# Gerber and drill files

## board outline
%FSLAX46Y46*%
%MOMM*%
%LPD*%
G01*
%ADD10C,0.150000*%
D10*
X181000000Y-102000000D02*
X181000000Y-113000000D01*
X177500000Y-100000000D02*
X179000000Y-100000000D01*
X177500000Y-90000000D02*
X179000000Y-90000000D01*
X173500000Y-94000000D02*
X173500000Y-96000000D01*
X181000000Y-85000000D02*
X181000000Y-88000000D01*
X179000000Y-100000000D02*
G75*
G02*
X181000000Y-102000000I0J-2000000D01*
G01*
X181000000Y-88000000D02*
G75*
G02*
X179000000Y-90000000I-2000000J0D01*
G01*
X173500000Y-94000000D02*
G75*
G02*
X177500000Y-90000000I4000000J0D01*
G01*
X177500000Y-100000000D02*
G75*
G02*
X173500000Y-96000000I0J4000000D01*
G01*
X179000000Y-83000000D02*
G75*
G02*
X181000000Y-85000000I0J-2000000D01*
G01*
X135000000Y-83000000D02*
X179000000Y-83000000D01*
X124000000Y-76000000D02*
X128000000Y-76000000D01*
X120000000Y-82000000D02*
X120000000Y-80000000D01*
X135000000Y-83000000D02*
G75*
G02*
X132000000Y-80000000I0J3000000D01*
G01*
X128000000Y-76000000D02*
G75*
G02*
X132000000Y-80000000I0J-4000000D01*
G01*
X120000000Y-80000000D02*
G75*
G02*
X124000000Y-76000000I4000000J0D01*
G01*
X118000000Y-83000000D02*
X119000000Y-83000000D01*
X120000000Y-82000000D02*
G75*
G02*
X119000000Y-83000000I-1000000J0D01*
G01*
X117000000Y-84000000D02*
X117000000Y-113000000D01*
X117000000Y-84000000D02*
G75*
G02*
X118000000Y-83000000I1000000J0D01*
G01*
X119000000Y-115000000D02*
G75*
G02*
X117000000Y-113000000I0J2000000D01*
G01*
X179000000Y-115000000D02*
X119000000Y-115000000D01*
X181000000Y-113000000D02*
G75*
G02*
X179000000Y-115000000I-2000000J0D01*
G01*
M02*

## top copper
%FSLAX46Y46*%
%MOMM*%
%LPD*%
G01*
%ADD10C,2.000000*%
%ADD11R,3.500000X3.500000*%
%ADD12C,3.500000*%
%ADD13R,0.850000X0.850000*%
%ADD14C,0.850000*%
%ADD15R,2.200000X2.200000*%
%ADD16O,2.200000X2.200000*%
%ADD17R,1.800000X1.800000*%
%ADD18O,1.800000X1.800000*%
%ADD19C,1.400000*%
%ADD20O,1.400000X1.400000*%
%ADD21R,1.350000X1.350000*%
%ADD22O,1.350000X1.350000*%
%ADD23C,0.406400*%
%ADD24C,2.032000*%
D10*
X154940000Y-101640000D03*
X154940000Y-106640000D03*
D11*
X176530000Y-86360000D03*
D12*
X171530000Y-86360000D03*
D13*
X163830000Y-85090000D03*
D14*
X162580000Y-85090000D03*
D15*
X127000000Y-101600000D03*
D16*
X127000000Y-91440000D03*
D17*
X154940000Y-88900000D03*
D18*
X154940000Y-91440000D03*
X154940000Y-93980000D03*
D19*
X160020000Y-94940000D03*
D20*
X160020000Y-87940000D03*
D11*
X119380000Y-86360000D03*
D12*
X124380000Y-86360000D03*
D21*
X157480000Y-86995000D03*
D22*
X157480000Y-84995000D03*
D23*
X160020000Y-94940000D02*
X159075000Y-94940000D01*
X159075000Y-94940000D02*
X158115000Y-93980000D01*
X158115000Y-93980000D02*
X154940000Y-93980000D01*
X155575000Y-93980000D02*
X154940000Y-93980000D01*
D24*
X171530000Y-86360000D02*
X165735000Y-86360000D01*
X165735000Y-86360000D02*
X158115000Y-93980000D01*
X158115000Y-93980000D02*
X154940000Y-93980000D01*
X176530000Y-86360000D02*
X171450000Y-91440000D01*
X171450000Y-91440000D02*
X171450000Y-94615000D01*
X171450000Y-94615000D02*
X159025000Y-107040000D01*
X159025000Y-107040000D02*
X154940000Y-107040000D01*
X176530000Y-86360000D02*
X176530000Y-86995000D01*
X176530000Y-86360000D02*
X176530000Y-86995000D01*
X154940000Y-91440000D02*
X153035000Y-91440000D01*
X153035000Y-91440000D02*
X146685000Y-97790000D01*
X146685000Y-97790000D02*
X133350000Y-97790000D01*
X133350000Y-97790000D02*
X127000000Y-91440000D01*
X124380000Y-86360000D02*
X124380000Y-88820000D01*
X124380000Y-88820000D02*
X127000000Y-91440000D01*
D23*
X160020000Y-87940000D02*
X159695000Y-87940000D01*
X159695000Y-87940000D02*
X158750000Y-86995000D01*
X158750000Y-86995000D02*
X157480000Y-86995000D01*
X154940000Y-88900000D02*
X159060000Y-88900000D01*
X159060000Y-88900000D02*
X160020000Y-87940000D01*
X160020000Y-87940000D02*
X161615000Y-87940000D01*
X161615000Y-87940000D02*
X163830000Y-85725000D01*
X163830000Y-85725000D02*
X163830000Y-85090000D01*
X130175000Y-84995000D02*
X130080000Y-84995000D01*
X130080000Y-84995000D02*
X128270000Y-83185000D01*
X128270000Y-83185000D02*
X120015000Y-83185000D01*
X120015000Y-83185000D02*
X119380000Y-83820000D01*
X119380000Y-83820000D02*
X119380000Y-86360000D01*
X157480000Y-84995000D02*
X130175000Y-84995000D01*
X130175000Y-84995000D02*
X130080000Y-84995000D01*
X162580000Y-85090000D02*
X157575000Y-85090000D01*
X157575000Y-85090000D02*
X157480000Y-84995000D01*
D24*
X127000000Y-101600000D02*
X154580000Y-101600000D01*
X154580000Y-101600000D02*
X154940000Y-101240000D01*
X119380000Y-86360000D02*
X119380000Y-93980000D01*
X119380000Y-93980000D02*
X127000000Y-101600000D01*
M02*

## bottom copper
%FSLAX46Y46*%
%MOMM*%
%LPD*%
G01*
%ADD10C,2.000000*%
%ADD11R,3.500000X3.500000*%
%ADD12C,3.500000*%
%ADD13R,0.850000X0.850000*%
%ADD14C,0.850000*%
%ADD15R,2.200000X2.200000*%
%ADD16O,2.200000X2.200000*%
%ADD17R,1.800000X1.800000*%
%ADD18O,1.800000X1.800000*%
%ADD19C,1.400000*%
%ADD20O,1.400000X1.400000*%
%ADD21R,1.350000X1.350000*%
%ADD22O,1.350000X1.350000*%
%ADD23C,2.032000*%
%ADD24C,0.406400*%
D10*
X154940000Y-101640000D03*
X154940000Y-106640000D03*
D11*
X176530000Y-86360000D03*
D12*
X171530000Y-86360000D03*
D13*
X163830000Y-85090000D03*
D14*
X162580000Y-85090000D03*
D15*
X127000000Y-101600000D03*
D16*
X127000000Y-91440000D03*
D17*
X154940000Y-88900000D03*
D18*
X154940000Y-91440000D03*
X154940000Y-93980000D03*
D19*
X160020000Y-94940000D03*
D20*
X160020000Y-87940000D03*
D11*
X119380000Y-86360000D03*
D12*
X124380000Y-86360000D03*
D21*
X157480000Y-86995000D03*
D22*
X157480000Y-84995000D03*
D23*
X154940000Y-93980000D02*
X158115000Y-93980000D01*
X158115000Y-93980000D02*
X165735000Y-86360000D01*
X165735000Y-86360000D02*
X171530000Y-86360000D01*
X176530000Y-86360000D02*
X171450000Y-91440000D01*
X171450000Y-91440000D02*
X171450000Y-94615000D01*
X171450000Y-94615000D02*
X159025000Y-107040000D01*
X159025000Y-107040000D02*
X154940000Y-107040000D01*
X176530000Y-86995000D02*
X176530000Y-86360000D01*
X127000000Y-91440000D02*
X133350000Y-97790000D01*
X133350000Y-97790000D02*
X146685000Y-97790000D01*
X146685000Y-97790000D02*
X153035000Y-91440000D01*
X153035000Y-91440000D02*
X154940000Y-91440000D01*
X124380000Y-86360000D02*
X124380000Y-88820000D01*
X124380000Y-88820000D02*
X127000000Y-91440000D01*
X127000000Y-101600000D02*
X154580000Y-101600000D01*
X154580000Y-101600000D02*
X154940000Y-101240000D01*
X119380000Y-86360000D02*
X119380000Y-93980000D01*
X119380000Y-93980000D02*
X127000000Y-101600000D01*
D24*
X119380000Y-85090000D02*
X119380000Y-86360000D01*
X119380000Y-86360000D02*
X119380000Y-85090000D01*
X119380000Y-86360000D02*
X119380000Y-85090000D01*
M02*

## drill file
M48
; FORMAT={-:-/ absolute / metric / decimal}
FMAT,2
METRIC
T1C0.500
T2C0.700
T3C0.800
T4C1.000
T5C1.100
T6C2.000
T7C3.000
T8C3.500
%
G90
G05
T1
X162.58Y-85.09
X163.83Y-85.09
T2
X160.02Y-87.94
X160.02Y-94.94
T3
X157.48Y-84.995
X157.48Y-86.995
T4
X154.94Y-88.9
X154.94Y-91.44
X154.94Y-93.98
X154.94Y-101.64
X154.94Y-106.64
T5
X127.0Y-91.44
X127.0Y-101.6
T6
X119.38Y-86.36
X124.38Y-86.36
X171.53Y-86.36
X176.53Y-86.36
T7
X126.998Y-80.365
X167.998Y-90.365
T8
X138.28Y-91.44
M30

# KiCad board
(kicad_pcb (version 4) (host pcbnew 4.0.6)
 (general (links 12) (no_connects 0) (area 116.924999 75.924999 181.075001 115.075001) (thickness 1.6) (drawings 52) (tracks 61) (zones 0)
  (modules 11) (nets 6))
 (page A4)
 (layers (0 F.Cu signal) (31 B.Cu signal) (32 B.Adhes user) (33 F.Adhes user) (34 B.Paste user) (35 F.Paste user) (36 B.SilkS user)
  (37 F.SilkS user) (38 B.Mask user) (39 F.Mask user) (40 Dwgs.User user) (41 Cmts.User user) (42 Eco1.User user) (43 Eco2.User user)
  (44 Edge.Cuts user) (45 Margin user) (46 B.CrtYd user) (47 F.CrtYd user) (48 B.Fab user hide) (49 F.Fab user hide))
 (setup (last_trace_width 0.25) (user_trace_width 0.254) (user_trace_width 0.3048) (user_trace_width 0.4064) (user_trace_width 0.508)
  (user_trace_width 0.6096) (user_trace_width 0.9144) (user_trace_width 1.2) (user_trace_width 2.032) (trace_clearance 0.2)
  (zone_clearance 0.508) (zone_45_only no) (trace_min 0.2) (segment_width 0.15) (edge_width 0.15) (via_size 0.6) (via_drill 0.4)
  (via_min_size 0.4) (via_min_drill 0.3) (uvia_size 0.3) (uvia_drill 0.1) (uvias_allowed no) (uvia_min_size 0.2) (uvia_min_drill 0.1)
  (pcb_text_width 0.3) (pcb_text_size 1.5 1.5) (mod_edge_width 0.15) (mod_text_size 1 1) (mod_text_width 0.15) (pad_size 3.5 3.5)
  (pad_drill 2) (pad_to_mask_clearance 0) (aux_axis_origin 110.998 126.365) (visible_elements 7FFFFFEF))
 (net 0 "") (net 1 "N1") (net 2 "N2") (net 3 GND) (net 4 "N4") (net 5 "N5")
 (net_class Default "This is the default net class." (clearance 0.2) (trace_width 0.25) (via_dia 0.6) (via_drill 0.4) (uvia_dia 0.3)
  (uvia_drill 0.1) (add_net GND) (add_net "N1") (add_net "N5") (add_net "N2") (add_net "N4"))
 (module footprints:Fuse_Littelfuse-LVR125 (layer B.Cu) (at 154.94 104.14 270)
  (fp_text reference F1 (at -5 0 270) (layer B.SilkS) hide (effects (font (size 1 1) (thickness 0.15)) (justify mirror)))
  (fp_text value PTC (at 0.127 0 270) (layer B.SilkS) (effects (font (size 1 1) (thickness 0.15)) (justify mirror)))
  (pad 1 thru_hole circle (at -2.5 0 270) (size 2 2) (drill 1) (layers *.Cu *.Mask) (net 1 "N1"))
  (pad 2 thru_hole circle (at 2.5 0 270) (size 2 2) (drill 1) (layers *.Cu *.Mask) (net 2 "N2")))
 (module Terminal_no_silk (layer B.Cu) (at 176.53 86.36 180)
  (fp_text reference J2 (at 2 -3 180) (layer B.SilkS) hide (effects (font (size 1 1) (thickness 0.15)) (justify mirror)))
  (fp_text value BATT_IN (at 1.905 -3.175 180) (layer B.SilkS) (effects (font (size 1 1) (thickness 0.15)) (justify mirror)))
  (pad 1 thru_hole rect (at 0 0 180) (size 3.5 3.5) (drill 2) (layers *.Cu *.Mask) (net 2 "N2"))
  (pad 2 thru_hole circle (at 5 0 180) (size 3.5 3.5) (drill 2) (layers *.Cu *.Mask) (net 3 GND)))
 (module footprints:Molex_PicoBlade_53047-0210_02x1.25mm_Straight (layer F.Cu) (at 163.83 85.09 180)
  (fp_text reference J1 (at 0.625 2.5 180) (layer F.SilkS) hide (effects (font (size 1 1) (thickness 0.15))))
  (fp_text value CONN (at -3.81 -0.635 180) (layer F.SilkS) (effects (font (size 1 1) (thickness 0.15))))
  (pad 1 thru_hole rect (at 0 0 180) (size 0.85 0.85) (drill 0.5) (layers *.Cu *.Mask) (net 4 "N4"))
  (pad 2 thru_hole circle (at 1.25 0 180) (size 0.85 0.85) (drill 0.5) (layers *.Cu *.Mask) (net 1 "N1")))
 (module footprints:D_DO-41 (layer B.Cu) (at 127 101.6 90)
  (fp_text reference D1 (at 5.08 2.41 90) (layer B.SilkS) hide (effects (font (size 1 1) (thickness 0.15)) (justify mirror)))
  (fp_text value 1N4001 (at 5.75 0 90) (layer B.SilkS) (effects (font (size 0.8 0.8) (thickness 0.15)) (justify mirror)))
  (pad 1 thru_hole rect (at 0 0 90) (size 2.2 2.2) (drill 1.1) (layers *.Cu *.Mask) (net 1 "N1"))
  (pad 2 thru_hole oval (at 10.16 0 90) (size 2.2 2.2) (drill 1.1) (layers *.Cu *.Mask) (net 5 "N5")))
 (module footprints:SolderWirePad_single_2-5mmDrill (layer F.Cu) (at 167.998 90.365)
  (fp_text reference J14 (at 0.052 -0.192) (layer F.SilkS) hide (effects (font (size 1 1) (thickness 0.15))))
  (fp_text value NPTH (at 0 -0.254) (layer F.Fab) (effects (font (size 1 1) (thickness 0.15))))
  (pad "" np_thru_hole circle (at 0 0) (size 3 3) (drill 3) (layers *.Cu *.Mask)))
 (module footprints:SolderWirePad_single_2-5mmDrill (layer F.Cu) (at 126.998 80.365)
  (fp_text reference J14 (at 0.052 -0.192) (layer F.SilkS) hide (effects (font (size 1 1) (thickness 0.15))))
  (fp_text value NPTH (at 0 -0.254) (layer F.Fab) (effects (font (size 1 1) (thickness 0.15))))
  (pad "" np_thru_hole circle (at 0 0) (size 3 3) (drill 3) (layers *.Cu *.Mask)))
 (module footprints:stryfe (layer F.Cu) (at 147.32 109.855)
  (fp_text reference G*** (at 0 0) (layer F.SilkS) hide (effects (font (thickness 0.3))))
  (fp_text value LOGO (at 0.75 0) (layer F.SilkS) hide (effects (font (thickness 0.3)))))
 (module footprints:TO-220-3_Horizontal (layer B.Cu) (at 154.94 88.9 270)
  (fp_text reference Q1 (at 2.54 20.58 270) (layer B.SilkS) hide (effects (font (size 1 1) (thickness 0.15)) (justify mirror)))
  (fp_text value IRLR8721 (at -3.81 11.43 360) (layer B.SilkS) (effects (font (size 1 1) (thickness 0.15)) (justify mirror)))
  (pad 0 np_thru_hole oval (at 2.54 16.66 270) (size 3.5 3.5) (drill 3.5) (layers *.Cu *.Mask))
  (pad 1 thru_hole rect (at 0 0 270) (size 1.8 1.8) (drill 1) (layers *.Cu *.Mask) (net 4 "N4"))
  (pad 2 thru_hole oval (at 2.54 0 270) (size 1.8 1.8) (drill 1) (layers *.Cu *.Mask) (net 5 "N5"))
  (pad 3 thru_hole oval (at 5.08 0 270) (size 1.8 1.8) (drill 1) (layers *.Cu *.Mask) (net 3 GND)))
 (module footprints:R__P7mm (layer B.Cu) (at 160.02 91.44 90)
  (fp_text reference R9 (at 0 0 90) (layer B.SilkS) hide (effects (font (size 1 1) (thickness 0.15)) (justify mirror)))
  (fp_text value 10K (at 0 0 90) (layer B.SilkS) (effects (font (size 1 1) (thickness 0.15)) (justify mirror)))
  (pad 1 thru_hole circle (at -3.5 0 90) (size 1.4 1.4) (drill 0.7) (layers *.Cu *.Mask) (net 3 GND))
  (pad 2 thru_hole oval (at 3.5 0 90) (size 1.4 1.4) (drill 0.7) (layers *.Cu *.Mask) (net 4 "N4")))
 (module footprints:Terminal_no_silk (layer B.Cu) (at 119.38 86.36)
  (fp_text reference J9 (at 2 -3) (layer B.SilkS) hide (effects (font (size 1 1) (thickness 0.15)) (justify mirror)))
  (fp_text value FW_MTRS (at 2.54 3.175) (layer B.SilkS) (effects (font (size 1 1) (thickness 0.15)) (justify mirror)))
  (pad 1 thru_hole rect (at 0 0) (size 3.5 3.5) (drill 2) (layers *.Cu *.Mask) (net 1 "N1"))
  (pad 2 thru_hole circle (at 5 0) (size 3.5 3.5) (drill 2) (layers *.Cu *.Mask) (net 5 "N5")))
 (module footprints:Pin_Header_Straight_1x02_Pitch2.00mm (layer F.Cu) (at 157.48 86.995 180)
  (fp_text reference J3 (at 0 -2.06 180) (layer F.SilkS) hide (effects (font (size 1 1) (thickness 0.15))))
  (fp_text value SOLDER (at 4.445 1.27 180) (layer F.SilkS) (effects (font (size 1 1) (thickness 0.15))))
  (pad 1 thru_hole rect (at 0 0 180) (size 1.35 1.35) (drill 0.8) (layers *.Cu *.Mask) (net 4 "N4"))
  (pad 2 thru_hole oval (at 0 2 180) (size 1.35 1.35) (drill 0.8) (layers *.Cu *.Mask) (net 1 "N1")))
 (gr_line (start 181 102) (end 181 113) (angle 90) (layer Edge.Cuts) (width 0.15))
 (gr_line (start 177.5 100) (end 179 100) (angle 90) (layer Edge.Cuts) (width 0.15))
 (gr_line (start 177.5 90) (end 179 90) (angle 90) (layer Edge.Cuts) (width 0.15))
 (gr_line (start 173.5 94) (end 173.5 96) (angle 90) (layer Edge.Cuts) (width 0.15))
 (gr_line (start 181 85) (end 181 88) (angle 90) (layer Edge.Cuts) (width 0.15))
 (gr_arc (start 179 102) (end 179 100) (angle 90) (layer Edge.Cuts) (width 0.15))
 (gr_arc (start 179 88) (end 181 88) (angle 90) (layer Edge.Cuts) (width 0.15))
 (gr_arc (start 177.5 94) (end 173.5 94) (angle 90) (layer Edge.Cuts) (width 0.15))
 (gr_arc (start 177.5 96) (end 177.5 100) (angle 90) (layer Edge.Cuts) (width 0.15))
 (gr_arc (start 179 85) (end 179 83) (angle 90) (layer Edge.Cuts) (width 0.15))
 (gr_line (start 135 83) (end 179 83) (angle 90) (layer Edge.Cuts) (width 0.15))
 (gr_line (start 124 76) (end 128 76) (angle 90) (layer Edge.Cuts) (width 0.15))
 (gr_line (start 120 82) (end 120 80) (angle 90) (layer Edge.Cuts) (width 0.15))
 (gr_arc (start 135 80) (end 135 83) (angle 90) (layer Edge.Cuts) (width 0.15))
 (gr_arc (start 128 80) (end 128 76) (angle 90) (layer Edge.Cuts) (width 0.15))
 (gr_arc (start 124 80) (end 120 80) (angle 90) (layer Edge.Cuts) (width 0.15))
 (gr_line (start 118 83) (end 119 83) (angle 90) (layer Edge.Cuts) (width 0.15))
 (gr_arc (start 119 82) (end 120 82) (angle 90) (layer Edge.Cuts) (width 0.15))
 (gr_line (start 117 84) (end 117 113) (angle 90) (layer Edge.Cuts) (width 0.15))
 (gr_arc (start 118 84) (end 117 84) (angle 90) (layer Edge.Cuts) (width 0.15))
 (gr_arc (start 119 113) (end 119 115) (angle 90) (layer Edge.Cuts) (width 0.15))
 (gr_line (start 179 115) (end 119 115) (angle 90) (layer Edge.Cuts) (width 0.15))
 (gr_arc (start 179 113) (end 181 113) (angle 90) (layer Edge.Cuts) (width 0.15))
 (segment (start 160.02 94.94) (end 159.075 94.94) (width 0.4064) (layer F.Cu) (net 3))
 (segment (start 159.075 94.94) (end 158.115 93.98) (width 0.4064) (layer F.Cu) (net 3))
 (segment (start 158.115 93.98) (end 154.94 93.98) (width 0.4064) (layer F.Cu) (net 3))
 (segment (start 155.575 93.98) (end 154.94 93.98) (width 0.4064) (layer F.Cu) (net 3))
 (segment (start 154.94 93.98) (end 158.115 93.98) (width 2.032) (layer B.Cu) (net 3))
 (segment (start 158.115 93.98) (end 165.735 86.36) (width 2.032) (layer B.Cu) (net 3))
 (segment (start 165.735 86.36) (end 171.53 86.36) (width 2.032) (layer B.Cu) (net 3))
 (segment (start 171.53 86.36) (end 165.735 86.36) (width 2.032) (layer F.Cu) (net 3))
 (segment (start 165.735 86.36) (end 158.115 93.98) (width 2.032) (layer F.Cu) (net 3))
 (segment (start 158.115 93.98) (end 154.94 93.98) (width 2.032) (layer F.Cu) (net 3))
 (segment (start 176.53 86.36) (end 171.45 91.44) (width 2.032) (layer B.Cu) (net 2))
 (segment (start 171.45 91.44) (end 171.45 94.615) (width 2.032) (layer B.Cu) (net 2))
 (segment (start 171.45 94.615) (end 159.025 107.04) (width 2.032) (layer B.Cu) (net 2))
 (segment (start 159.025 107.04) (end 154.94 107.04) (width 2.032) (layer B.Cu) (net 2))
 (segment (start 176.53 86.36) (end 171.45 91.44) (width 2.032) (layer F.Cu) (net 2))
 (segment (start 171.45 91.44) (end 171.45 94.615) (width 2.032) (layer F.Cu) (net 2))
 (segment (start 171.45 94.615) (end 159.025 107.04) (width 2.032) (layer F.Cu) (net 2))
 (segment (start 159.025 107.04) (end 154.94 107.04) (width 2.032) (layer F.Cu) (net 2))
 (segment (start 176.53 86.995) (end 176.53 86.36) (width 2.032) (layer B.Cu) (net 2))
 (segment (start 176.53 86.36) (end 176.53 86.995) (width 2.032) (layer F.Cu) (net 2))
 (segment (start 176.53 86.36) (end 176.53 86.995) (width 2.032) (layer F.Cu) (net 2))
 (segment (start 127 91.44) (end 133.35 97.79) (width 2.032) (layer B.Cu) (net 5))
 (segment (start 133.35 97.79) (end 146.685 97.79) (width 2.032) (layer B.Cu) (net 5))
 (segment (start 146.685 97.79) (end 153.035 91.44) (width 2.032) (layer B.Cu) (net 5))
 (segment (start 153.035 91.44) (end 154.94 91.44) (width 2.032) (layer B.Cu) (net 5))
 (segment (start 154.94 91.44) (end 153.035 91.44) (width 2.032) (layer F.Cu) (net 5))
 (segment (start 153.035 91.44) (end 146.685 97.79) (width 2.032) (layer F.Cu) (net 5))
 (segment (start 146.685 97.79) (end 133.35 97.79) (width 2.032) (layer F.Cu) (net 5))
 (segment (start 133.35 97.79) (end 127 91.44) (width 2.032) (layer F.Cu) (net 5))
 (segment (start 124.38 86.36) (end 124.38 88.82) (width 2.032) (layer B.Cu) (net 5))
 (segment (start 124.38 88.82) (end 127 91.44) (width 2.032) (layer B.Cu) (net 5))
 (segment (start 124.38 86.36) (end 124.38 88.82) (width 2.032) (layer F.Cu) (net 5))
 (segment (start 124.38 88.82) (end 127 91.44) (width 2.032) (layer F.Cu) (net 5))
 (segment (start 160.02 87.94) (end 159.695 87.94) (width 0.4064) (layer F.Cu) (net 4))
 (segment (start 159.695 87.94) (end 158.75 86.995) (width 0.4064) (layer F.Cu) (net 4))
 (segment (start 158.75 86.995) (end 157.48 86.995) (width 0.4064) (layer F.Cu) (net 4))
 (segment (start 154.94 88.9) (end 159.06 88.9) (width 0.4064) (layer F.Cu) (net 4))
 (segment (start 159.06 88.9) (end 160.02 87.94) (width 0.4064) (layer F.Cu) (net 4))
 (segment (start 160.02 87.94) (end 161.615 87.94) (width 0.4064) (layer F.Cu) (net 4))
 (segment (start 161.615 87.94) (end 163.83 85.725) (width 0.4064) (layer F.Cu) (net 4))
 (segment (start 163.83 85.725) (end 163.83 85.09) (width 0.4064) (layer F.Cu) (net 4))
 (segment (start 130.175 84.995) (end 130.08 84.995) (width 0.4064) (layer F.Cu) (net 1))
 (segment (start 130.08 84.995) (end 128.27 83.185) (width 0.4064) (layer F.Cu) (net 1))
 (segment (start 128.27 83.185) (end 120.015 83.185) (width 0.4064) (layer F.Cu) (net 1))
 (segment (start 120.015 83.185) (end 119.38 83.82) (width 0.4064) (layer F.Cu) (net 1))
 (segment (start 119.38 83.82) (end 119.38 86.36) (width 0.4064) (layer F.Cu) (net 1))
 (segment (start 157.48 84.995) (end 130.175 84.995) (width 0.4064) (layer F.Cu) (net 1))
 (segment (start 130.175 84.995) (end 130.08 84.995) (width 0.4064) (layer F.Cu) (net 1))
 (segment (start 162.58 85.09) (end 157.575 85.09) (width 0.4064) (layer F.Cu) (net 1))
 (segment (start 157.575 85.09) (end 157.48 84.995) (width 0.4064) (layer F.Cu) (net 1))
 (segment (start 127 101.6) (end 154.58 101.6) (width 2.032) (layer F.Cu) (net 1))
 (segment (start 154.58 101.6) (end 154.94 101.24) (width 2.032) (layer F.Cu) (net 1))
 (segment (start 127 101.6) (end 154.58 101.6) (width 2.032) (layer B.Cu) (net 1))
 (segment (start 154.58 101.6) (end 154.94 101.24) (width 2.032) (layer B.Cu) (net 1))
 (segment (start 119.38 86.36) (end 119.38 93.98) (width 2.032) (layer B.Cu) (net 1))
 (segment (start 119.38 93.98) (end 127 101.6) (width 2.032) (layer B.Cu) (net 1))
 (segment (start 119.38 86.36) (end 119.38 93.98) (width 2.032) (layer F.Cu) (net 1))
 (segment (start 119.38 93.98) (end 127 101.6) (width 2.032) (layer F.Cu) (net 1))
 (segment (start 119.38 85.09) (end 119.38 86.36) (width 0.4064) (layer B.Cu) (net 1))
 (segment (start 119.38 86.36) (end 119.38 85.09) (width 0.4064) (layer B.Cu) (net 1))
 (segment (start 119.38 86.36) (end 119.38 85.09) (width 0.4064) (layer B.Cu) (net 1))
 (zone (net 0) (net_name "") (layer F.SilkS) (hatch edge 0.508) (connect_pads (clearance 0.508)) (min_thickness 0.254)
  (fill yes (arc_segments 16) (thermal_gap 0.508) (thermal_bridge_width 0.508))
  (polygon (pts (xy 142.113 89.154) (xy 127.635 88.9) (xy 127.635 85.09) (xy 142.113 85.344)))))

